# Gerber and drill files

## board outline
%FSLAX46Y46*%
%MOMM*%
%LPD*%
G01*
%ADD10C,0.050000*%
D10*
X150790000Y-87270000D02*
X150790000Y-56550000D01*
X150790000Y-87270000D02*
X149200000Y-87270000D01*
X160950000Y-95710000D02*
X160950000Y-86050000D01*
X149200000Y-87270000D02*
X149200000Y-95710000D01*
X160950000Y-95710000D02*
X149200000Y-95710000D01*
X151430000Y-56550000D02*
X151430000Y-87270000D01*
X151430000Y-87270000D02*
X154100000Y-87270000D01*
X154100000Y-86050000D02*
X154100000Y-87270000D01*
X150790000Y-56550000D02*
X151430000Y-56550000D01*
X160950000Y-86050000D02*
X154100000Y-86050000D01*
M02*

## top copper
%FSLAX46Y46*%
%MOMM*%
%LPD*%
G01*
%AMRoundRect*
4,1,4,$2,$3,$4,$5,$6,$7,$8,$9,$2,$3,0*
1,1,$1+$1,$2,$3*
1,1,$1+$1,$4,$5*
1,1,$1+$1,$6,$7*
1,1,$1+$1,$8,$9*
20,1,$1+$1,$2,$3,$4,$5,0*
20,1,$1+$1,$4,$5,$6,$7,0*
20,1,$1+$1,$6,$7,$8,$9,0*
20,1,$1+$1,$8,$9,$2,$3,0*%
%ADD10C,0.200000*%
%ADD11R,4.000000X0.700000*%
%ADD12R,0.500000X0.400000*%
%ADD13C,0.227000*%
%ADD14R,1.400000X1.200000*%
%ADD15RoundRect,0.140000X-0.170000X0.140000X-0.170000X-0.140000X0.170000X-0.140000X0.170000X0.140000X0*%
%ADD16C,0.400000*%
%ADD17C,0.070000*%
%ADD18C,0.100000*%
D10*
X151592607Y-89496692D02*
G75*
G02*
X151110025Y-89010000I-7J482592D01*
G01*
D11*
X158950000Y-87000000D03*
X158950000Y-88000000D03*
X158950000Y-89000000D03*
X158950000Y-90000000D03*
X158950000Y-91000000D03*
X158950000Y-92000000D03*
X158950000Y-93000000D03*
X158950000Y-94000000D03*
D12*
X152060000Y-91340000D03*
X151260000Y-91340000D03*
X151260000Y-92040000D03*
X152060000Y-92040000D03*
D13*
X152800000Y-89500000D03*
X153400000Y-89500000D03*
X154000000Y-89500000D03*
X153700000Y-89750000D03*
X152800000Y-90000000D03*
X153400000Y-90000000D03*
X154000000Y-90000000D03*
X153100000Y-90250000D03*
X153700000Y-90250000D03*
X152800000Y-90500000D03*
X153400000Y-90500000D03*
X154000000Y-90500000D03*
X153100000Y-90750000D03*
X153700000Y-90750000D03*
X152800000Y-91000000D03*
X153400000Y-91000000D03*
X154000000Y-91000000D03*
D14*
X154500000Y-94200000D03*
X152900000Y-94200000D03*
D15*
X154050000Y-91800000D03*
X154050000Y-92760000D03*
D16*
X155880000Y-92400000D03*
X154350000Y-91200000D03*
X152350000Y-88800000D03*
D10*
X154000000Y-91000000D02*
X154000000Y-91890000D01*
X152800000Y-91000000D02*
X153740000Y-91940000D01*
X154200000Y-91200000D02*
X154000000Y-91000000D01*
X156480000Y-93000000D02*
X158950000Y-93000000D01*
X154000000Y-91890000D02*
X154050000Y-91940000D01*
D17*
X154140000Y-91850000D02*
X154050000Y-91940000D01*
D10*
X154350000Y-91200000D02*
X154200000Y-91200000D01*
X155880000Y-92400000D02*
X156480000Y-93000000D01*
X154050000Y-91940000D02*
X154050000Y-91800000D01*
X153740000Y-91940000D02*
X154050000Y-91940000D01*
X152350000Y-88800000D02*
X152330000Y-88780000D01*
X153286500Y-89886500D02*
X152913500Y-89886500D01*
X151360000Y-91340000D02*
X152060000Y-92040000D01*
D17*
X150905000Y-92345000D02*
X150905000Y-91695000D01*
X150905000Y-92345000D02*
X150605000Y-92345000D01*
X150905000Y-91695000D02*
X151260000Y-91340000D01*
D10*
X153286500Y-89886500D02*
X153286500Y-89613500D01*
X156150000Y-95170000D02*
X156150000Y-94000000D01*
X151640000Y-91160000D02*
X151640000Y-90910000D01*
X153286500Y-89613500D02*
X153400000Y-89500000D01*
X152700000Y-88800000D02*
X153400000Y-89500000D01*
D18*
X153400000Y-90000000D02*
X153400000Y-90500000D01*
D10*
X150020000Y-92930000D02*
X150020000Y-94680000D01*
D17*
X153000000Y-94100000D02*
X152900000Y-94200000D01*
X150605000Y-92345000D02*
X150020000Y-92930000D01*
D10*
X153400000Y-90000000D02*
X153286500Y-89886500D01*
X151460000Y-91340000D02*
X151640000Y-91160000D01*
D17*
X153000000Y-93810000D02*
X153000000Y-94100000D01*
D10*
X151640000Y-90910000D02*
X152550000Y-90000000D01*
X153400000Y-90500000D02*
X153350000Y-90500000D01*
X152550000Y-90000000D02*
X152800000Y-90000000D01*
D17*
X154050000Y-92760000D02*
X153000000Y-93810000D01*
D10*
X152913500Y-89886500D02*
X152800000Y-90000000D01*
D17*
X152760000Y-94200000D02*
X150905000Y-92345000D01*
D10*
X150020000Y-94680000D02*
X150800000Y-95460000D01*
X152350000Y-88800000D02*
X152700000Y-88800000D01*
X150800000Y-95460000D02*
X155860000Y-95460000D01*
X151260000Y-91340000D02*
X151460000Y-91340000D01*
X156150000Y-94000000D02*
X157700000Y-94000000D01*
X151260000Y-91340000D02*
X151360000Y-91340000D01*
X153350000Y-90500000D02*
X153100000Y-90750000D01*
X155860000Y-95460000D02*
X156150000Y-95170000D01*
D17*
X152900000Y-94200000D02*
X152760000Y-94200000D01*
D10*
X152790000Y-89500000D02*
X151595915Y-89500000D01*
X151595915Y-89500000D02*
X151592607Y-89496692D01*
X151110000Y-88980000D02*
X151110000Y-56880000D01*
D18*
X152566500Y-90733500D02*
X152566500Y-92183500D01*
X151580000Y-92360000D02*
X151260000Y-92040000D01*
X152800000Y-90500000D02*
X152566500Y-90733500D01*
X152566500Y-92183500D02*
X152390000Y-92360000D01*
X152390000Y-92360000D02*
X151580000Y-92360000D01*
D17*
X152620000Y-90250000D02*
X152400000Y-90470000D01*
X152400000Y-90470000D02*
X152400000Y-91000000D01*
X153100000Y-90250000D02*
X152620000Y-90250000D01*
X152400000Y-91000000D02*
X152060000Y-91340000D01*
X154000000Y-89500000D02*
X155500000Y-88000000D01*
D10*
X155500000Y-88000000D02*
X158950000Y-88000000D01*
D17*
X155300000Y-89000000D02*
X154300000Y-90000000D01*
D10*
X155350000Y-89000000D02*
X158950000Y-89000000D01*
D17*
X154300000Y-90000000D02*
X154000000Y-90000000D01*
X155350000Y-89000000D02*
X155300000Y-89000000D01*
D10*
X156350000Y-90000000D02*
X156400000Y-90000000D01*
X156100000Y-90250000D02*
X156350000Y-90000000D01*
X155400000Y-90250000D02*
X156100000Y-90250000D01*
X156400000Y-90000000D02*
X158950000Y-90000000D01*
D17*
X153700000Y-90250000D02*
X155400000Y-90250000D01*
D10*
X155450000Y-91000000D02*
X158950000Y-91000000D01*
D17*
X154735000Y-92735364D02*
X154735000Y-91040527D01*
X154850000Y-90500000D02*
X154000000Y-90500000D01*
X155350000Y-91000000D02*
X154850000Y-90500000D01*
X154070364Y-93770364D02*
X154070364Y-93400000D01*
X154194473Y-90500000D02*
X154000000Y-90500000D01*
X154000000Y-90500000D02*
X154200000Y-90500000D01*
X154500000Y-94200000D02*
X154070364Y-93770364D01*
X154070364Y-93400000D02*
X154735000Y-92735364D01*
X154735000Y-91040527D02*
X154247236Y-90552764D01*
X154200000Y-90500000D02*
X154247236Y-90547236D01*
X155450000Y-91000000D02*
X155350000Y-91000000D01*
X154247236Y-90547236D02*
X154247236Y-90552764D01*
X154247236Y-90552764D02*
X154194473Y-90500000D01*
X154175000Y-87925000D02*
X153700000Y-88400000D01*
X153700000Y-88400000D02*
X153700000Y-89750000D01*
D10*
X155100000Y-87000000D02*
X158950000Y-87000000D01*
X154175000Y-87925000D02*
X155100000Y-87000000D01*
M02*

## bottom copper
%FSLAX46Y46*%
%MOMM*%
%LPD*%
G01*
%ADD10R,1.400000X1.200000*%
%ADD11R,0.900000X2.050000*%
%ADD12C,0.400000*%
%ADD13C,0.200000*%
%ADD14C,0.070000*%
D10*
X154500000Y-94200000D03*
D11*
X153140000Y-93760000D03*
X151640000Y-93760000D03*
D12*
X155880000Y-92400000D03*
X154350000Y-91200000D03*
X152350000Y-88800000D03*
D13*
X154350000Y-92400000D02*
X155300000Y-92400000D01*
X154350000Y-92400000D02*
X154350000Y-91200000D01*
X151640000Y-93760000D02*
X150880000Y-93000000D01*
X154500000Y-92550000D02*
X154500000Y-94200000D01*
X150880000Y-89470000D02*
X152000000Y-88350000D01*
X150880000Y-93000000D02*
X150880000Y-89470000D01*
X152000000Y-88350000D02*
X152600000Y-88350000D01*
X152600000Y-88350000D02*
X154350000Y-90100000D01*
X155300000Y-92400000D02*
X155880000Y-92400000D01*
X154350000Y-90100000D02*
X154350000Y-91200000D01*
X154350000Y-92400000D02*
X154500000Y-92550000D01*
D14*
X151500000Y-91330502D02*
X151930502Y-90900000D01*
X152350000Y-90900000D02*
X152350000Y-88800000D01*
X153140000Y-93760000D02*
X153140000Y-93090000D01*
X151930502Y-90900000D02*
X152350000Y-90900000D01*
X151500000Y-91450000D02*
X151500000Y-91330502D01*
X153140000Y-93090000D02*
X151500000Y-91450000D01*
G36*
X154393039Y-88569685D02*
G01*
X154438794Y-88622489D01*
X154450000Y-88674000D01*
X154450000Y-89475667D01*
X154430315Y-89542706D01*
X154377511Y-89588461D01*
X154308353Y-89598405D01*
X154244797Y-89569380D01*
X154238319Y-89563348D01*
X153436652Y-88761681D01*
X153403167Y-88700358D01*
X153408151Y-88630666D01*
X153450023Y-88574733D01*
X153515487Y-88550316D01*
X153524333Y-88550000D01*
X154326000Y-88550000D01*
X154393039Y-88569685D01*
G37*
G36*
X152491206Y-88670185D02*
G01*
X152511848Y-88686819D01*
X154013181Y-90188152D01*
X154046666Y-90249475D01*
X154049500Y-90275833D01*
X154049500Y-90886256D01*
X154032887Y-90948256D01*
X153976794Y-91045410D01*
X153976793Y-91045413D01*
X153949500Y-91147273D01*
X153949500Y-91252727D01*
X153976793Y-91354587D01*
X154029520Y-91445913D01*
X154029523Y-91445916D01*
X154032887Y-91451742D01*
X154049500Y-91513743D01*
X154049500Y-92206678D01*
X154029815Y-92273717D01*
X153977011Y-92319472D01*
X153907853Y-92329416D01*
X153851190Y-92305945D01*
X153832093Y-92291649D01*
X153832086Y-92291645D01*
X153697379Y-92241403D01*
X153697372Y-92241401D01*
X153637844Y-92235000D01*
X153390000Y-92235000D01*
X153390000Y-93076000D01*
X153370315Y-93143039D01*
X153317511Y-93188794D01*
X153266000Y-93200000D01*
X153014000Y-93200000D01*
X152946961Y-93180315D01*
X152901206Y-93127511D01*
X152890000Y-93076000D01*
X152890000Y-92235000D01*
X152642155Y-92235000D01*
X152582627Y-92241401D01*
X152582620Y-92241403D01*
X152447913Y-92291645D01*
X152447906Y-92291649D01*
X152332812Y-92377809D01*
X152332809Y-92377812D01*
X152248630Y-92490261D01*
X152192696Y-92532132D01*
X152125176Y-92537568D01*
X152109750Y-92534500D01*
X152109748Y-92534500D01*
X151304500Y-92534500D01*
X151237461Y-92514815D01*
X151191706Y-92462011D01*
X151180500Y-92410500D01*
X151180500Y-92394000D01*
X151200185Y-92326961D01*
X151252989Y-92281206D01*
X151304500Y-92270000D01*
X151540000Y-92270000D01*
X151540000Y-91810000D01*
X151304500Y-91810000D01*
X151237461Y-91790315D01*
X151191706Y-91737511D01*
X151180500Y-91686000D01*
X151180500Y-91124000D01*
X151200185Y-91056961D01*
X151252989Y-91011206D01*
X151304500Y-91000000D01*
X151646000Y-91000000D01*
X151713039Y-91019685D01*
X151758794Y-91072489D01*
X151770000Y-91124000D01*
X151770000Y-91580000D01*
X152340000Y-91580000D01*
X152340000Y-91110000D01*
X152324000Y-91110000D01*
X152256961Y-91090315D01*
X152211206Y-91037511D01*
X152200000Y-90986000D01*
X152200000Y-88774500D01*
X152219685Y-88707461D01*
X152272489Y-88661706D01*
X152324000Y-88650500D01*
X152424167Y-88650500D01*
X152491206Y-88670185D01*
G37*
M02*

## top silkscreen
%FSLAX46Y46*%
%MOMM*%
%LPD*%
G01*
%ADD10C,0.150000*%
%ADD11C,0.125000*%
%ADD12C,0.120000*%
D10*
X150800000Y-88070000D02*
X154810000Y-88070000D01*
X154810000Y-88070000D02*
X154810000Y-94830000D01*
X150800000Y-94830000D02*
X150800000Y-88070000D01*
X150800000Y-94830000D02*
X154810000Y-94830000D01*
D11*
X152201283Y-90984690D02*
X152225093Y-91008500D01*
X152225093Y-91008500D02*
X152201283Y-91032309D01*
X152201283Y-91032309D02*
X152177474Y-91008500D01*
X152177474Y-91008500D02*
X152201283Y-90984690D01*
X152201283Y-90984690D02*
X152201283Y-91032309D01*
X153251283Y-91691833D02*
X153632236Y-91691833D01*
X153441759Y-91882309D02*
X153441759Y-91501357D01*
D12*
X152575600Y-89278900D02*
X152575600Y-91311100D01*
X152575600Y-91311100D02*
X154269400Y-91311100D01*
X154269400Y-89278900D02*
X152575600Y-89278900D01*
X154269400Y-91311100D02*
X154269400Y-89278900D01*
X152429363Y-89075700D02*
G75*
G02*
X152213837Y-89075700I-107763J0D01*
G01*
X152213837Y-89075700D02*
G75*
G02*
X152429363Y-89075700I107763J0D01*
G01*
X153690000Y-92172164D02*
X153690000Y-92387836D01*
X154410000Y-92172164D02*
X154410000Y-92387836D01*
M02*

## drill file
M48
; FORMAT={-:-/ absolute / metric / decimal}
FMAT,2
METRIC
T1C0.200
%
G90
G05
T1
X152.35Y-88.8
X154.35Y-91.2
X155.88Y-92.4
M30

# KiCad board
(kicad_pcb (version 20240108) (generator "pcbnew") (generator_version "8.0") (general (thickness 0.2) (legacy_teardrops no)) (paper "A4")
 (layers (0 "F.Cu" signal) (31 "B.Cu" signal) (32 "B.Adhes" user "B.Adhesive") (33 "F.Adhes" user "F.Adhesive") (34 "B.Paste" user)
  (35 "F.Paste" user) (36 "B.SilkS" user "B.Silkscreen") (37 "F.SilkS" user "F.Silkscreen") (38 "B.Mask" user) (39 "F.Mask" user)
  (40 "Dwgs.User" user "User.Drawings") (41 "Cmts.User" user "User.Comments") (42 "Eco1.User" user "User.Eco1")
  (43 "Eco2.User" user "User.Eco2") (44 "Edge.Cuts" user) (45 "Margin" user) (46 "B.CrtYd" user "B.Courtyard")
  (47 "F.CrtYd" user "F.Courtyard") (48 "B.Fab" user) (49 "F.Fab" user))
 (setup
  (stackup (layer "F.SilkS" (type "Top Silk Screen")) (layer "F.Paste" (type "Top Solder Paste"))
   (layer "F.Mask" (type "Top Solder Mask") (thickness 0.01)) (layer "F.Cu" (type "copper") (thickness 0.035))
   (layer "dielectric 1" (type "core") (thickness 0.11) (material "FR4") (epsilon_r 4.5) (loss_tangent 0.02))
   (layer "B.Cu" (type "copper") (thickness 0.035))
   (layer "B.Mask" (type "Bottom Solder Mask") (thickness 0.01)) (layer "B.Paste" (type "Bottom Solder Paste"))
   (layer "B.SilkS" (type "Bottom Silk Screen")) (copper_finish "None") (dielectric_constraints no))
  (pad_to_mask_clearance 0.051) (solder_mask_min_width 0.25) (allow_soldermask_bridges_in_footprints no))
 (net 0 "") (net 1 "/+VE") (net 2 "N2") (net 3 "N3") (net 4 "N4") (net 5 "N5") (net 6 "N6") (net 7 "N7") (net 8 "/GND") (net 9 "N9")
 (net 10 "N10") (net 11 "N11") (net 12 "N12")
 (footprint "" (layer "F.Cu") (at 154.5 94.2)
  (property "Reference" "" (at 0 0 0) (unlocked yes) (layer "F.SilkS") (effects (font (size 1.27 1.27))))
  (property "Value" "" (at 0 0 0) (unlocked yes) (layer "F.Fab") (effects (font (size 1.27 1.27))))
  (pad "2" smd rect (at 0 0 270) (size 1.2 1.4) (layers "B.Cu" "B.Paste" "B.Mask") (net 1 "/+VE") (solder_mask_margin 0.102)))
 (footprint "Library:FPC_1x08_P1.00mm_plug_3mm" (layer "F.Cu") (at 156.95 90.5)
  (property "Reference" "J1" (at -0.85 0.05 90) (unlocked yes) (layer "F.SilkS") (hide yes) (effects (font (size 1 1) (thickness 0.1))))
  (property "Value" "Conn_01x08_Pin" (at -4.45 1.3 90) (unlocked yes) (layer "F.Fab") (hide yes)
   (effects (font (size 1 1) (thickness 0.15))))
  (pad "1" connect rect (at 2 -3.5) (size 4 0.7) (layers "F.Cu" "F.Mask") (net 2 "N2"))
  (pad "2" connect rect (at 2 -2.5) (size 4 0.7) (layers "F.Cu" "F.Mask") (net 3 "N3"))
  (pad "3" connect rect (at 2 -1.5) (size 4 0.7) (layers "F.Cu" "F.Mask") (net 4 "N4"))
  (pad "4" connect rect (at 2 -0.5) (size 4 0.7) (layers "F.Cu" "F.Mask") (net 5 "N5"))
  (pad "5" connect rect (at 2 0.5) (size 4 0.7) (layers "F.Cu" "F.Mask") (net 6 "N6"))
  (pad "6" connect rect (at 2 1.5) (size 4 0.7) (layers "F.Cu" "F.Mask") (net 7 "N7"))
  (pad "7" connect rect (at 2 2.5) (size 4 0.7) (layers "F.Cu" "F.Mask") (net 1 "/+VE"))
  (pad "8" connect rect (at 2 3.5) (size 4 0.7) (layers "F.Cu" "F.Mask") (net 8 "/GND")))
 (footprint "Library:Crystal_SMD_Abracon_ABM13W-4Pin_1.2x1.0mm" (layer "F.Cu") (at 151.66 91.69 180)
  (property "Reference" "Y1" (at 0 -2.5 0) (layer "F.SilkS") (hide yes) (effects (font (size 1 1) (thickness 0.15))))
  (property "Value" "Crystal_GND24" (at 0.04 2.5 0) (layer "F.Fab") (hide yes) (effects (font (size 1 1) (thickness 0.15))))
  (pad "1" smd rect (at -0.4 0.35 180) (size 0.5 0.4) (layers "F.Cu" "F.Paste" "F.Mask") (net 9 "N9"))
  (pad "2" smd rect (at 0.4 0.35 180) (size 0.5 0.4) (layers "F.Cu" "F.Paste" "F.Mask") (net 8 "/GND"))
  (pad "3" smd rect (at 0.4 -0.35 180) (size 0.5 0.4) (layers "F.Cu" "F.Paste" "F.Mask") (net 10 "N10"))
  (pad "4" smd rect (at -0.4 -0.35 180) (size 0.5 0.4) (layers "F.Cu" "F.Paste" "F.Mask") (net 8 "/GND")))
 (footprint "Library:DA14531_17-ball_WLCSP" (layer "F.Cu") (at 153.422 90.295)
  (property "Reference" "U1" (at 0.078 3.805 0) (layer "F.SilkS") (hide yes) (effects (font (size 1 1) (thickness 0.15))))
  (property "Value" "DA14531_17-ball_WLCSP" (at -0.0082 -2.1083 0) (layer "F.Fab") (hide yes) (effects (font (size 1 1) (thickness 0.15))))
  (fp_line (start -0.8464 -1.0161) (end -0.8464 1.0161) (stroke (width 0.12) (type solid)) (layer "F.SilkS"))
  (fp_line (start -0.8464 1.0161) (end 0.8474 1.0161) (stroke (width 0.12) (type solid)) (layer "F.SilkS"))
  (fp_line (start 0.8474 -1.0161) (end -0.8464 -1.0161) (stroke (width 0.12) (type solid)) (layer "F.SilkS"))
  (fp_line (start 0.8474 1.0161) (end 0.8474 -1.0161) (stroke (width 0.12) (type solid)) (layer "F.SilkS"))
  (fp_circle (center -1.1004 -1.2193) (end -1.0242 -1.1431) (stroke (width 0.12) (type solid)) (fill none) (layer "F.SilkS"))
  (pad "A1" smd circle (at -0.622 -0.795) (size 0.227 0.227) (layers "F.Cu" "F.Paste" "F.Mask") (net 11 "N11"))
  (pad "A3" smd circle (at -0.022 -0.795) (size 0.227 0.227) (layers "F.Cu" "F.Paste" "F.Mask") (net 8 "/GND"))
  (pad "A5" smd circle (at 0.578 -0.795) (size 0.227 0.227) (layers "F.Cu" "F.Paste" "F.Mask") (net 3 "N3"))
  (pad "B4" smd circle (at 0.278 -0.545) (size 0.227 0.227) (layers "F.Cu" "F.Paste" "F.Mask") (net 2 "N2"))
  (pad "C1" smd circle (at -0.622 -0.295) (size 0.227 0.227) (layers "F.Cu" "F.Paste" "F.Mask") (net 8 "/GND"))
  (pad "C3" smd circle (at -0.022 -0.295) (size 0.227 0.227) (layers "F.Cu" "F.Paste" "F.Mask") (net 8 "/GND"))
  (pad "C5" smd circle (at 0.578 -0.295) (size 0.227 0.227) (layers "F.Cu" "F.Paste" "F.Mask") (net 4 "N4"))
  (pad "D2" smd circle (at -0.322 -0.045) (size 0.227 0.227) (layers "F.Cu" "F.Paste" "F.Mask") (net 9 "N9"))
  (pad "D4" smd circle (at 0.278 -0.045) (size 0.227 0.227) (layers "F.Cu" "F.Paste" "F.Mask") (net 5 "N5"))
  (pad "E1" smd circle (at -0.622 0.205) (size 0.227 0.227) (layers "F.Cu" "F.Paste" "F.Mask") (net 10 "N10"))
  (pad "E3" smd circle (at -0.022 0.205) (size 0.227 0.227) (layers "F.Cu" "F.Paste" "F.Mask") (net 8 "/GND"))
  (pad "E5" smd circle (at 0.578 0.205) (size 0.227 0.227) (layers "F.Cu" "F.Paste" "F.Mask") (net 6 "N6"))
  (pad "F2" smd circle (at -0.322 0.455) (size 0.227 0.227) (layers "F.Cu" "F.Paste" "F.Mask") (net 8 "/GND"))
  (pad "F4" smd circle (at 0.278 0.455) (size 0.227 0.227) (layers "F.Cu" "F.Paste" "F.Mask") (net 7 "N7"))
  (pad "G1" smd circle (at -0.622 0.705) (size 0.227 0.227) (layers "F.Cu" "F.Paste" "F.Mask") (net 1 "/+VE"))
  (pad "G3" smd circle (at -0.022 0.705) (size 0.227 0.227) (layers "F.Cu" "F.Paste" "F.Mask") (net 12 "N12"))
  (pad "G5" smd circle (at 0.578 0.705) (size 0.227 0.227) (layers "F.Cu" "F.Paste" "F.Mask") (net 1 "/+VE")))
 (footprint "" (layer "F.Cu") (at 154.5 94.2)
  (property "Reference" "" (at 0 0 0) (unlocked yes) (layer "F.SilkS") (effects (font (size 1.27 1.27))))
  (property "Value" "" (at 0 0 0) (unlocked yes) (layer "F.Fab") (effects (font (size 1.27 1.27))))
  (pad "2" smd rect (at 0 0 270) (size 1.2 1.4) (layers "F.Cu" "F.Paste" "F.Mask") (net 6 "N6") (solder_mask_margin 0.102)))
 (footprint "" (layer "F.Cu") (at 152.9 94.2)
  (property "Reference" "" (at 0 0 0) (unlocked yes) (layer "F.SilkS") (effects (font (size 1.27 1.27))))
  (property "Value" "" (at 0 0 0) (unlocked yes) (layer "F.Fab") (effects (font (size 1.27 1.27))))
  (pad "2" smd rect (at 0 0 270) (size 1.2 1.4) (layers "F.Cu" "F.Paste" "F.Mask") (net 8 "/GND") (solder_mask_margin 0.102)))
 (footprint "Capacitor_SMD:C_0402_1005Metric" (layer "F.Cu") (at 154.05 92.28 -90)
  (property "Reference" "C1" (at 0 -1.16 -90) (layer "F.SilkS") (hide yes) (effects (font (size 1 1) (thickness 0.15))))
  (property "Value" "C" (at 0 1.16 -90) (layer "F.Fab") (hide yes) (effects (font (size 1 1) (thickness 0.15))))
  (fp_line (start -0.107836 0.36) (end 0.107836 0.36) (stroke (width 0.12) (type solid)) (layer "F.SilkS"))
  (fp_line (start -0.107836 -0.36) (end 0.107836 -0.36) (stroke (width 0.12) (type solid)) (layer "F.SilkS"))
  (pad "1" smd roundrect (at -0.48 0 270) (size 0.56 0.62) (layers "F.Cu" "F.Paste" "F.Mask") (roundrect_rratio 0.25) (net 1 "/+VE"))
  (pad "2" smd roundrect (at 0.48 0 270) (size 0.56 0.62) (layers "F.Cu" "F.Paste" "F.Mask") (roundrect_rratio 0.25) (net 8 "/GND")))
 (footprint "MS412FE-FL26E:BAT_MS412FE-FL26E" (layer "B.Cu") (at 152.39 90.035 -90)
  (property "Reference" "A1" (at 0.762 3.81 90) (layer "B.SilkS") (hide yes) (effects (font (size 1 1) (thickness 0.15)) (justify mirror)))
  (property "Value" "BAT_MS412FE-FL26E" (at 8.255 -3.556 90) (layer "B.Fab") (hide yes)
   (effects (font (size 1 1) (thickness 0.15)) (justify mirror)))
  (pad "N1" smd rect (at 3.725 -0.75 270) (size 2.05 0.9) (layers "B.Cu" "B.Paste" "B.Mask") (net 8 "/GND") (solder_mask_margin 0.102))
  (pad "P1" smd rect (at 3.725 0.75 270) (size 2.05 0.9) (layers "B.Cu" "B.Paste" "B.Mask") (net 1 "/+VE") (solder_mask_margin 0.102)))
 (gr_arc (start 151.592607 89.496692) (mid 151.249908 89.353892) (end 151.11 89.01) (stroke (width 0.2) (type default)) (layer "F.Cu")
  (net 11))
 (gr_line (start 150.8 88.07) (end 154.81 88.07) (stroke (width 0.15) (type default)) (layer "F.SilkS"))
 (gr_line (start 154.81 88.07) (end 154.81 94.83) (stroke (width 0.15) (type default)) (layer "F.SilkS"))
 (gr_line (start 150.8 94.83) (end 150.8 88.07) (stroke (width 0.15) (type default)) (layer "F.SilkS"))
 (gr_line (start 150.8 94.83) (end 154.81 94.83) (stroke (width 0.15) (type default)) (layer "F.SilkS"))
 (gr_line (start 150.79 87.27) (end 150.79 56.55) (stroke (width 0.05) (type default)) (layer "Edge.Cuts"))
 (gr_line (start 150.79 87.27) (end 149.2 87.27) (stroke (width 0.05) (type default)) (layer "Edge.Cuts"))
 (gr_line (start 160.95 95.71) (end 160.95 86.05) (stroke (width 0.05) (type default)) (layer "Edge.Cuts"))
 (gr_line (start 149.2 87.27) (end 149.2 95.71) (stroke (width 0.05) (type default)) (layer "Edge.Cuts"))
 (gr_line (start 160.95 95.71) (end 149.2 95.71) (stroke (width 0.05) (type default)) (layer "Edge.Cuts"))
 (gr_line (start 151.43 56.55) (end 151.43 87.27) (stroke (width 0.05) (type default)) (layer "Edge.Cuts"))
 (gr_line (start 151.43 87.27) (end 154.1 87.27) (stroke (width 0.05) (type default)) (layer "Edge.Cuts"))
 (gr_line (start 154.1 86.05) (end 154.1 87.27) (stroke (width 0.05) (type default)) (layer "Edge.Cuts"))
 (gr_line (start 150.79 56.55) (end 151.43 56.55) (stroke (width 0.05) (type default)) (layer "Edge.Cuts"))
 (gr_line (start 160.95 86.05) (end 154.1 86.05) (stroke (width 0.05) (type default)) (layer "Edge.Cuts"))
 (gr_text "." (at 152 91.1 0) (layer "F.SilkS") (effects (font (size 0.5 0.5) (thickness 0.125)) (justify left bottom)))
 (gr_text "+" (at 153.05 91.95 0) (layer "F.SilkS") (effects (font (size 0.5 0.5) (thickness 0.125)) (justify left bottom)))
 (segment (start 154 91) (end 154 91.89) (width 0.2) (layer "F.Cu") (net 1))
 (segment (start 152.8 91) (end 153.74 91.94) (width 0.2) (layer "F.Cu") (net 1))
 (segment (start 154.2 91.2) (end 154 91) (width 0.2) (layer "F.Cu") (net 1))
 (segment (start 156.48 93) (end 158.95 93) (width 0.2) (layer "F.Cu") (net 1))
 (segment (start 154 91.89) (end 154.05 91.94) (width 0.2) (layer "F.Cu") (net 1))
 (segment (start 154.14 91.85) (end 154.05 91.94) (width 0.07) (layer "F.Cu") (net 1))
 (segment (start 154.35 91.2) (end 154.2 91.2) (width 0.2) (layer "F.Cu") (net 1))
 (segment (start 155.88 92.4) (end 156.48 93) (width 0.2) (layer "F.Cu") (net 1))
 (segment (start 154.05 91.94) (end 154.05 91.8) (width 0.2) (layer "F.Cu") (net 1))
 (segment (start 153.74 91.94) (end 154.05 91.94) (width 0.2) (layer "F.Cu") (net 1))
 (via (at 155.88 92.4) (size 0.4) (drill 0.2) (layers "F.Cu" "B.Cu") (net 1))
 (via (at 154.35 91.2) (size 0.4) (drill 0.2) (layers "F.Cu" "B.Cu") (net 1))
 (segment (start 154.35 92.4) (end 155.3 92.4) (width 0.2) (layer "B.Cu") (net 1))
 (segment (start 154.35 92.4) (end 154.35 91.2) (width 0.2) (layer "B.Cu") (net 1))
 (segment (start 151.64 93.76) (end 150.88 93) (width 0.2) (layer "B.Cu") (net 1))
 (segment (start 154.5 92.55) (end 154.5 94.2) (width 0.2) (layer "B.Cu") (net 1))
 (segment (start 150.88 89.47) (end 152 88.35) (width 0.2) (layer "B.Cu") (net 1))
 (segment (start 150.88 93) (end 150.88 89.47) (width 0.2) (layer "B.Cu") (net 1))
 (segment (start 152 88.35) (end 152.6 88.35) (width 0.2) (layer "B.Cu") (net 1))
 (segment (start 152.6 88.35) (end 154.35 90.1) (width 0.2) (layer "B.Cu") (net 1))
 (segment (start 155.3 92.4) (end 155.88 92.4) (width 0.2) (layer "B.Cu") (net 1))
 (segment (start 154.35 90.1) (end 154.35 91.2) (width 0.2) (layer "B.Cu") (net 1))
 (segment (start 154.35 92.4) (end 154.5 92.55) (width 0.2) (layer "B.Cu") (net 1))
 (segment (start 152.35 88.8) (end 152.33 88.78) (width 0.2) (layer "F.Cu") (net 8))
 (segment (start 153.2865 89.8865) (end 152.9135 89.8865) (width 0.2) (layer "F.Cu") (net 8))
 (segment (start 151.36 91.34) (end 152.06 92.04) (width 0.2) (layer "F.Cu") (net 8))
 (segment (start 150.905 92.345) (end 150.905 91.695) (width 0.07) (layer "F.Cu") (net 8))
 (segment (start 150.905 92.345) (end 150.605 92.345) (width 0.07) (layer "F.Cu") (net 8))
 (segment (start 150.905 91.695) (end 151.26 91.34) (width 0.07) (layer "F.Cu") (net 8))
 (segment (start 153.2865 89.8865) (end 153.2865 89.6135) (width 0.2) (layer "F.Cu") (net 8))
 (segment (start 156.15 95.17) (end 156.15 94) (width 0.2) (layer "F.Cu") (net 8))
 (segment (start 151.64 91.16) (end 151.64 90.91) (width 0.2) (layer "F.Cu") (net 8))
 (segment (start 153.2865 89.6135) (end 153.4 89.5) (width 0.2) (layer "F.Cu") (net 8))
 (segment (start 152.7 88.8) (end 153.4 89.5) (width 0.2) (layer "F.Cu") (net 8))
 (segment (start 153.4 90) (end 153.4 90.5) (width 0.1) (layer "F.Cu") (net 8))
 (segment (start 150.02 92.93) (end 150.02 94.68) (width 0.2) (layer "F.Cu") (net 8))
 (segment (start 153 94.1) (end 152.9 94.2) (width 0.07) (layer "F.Cu") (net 8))
 (segment (start 150.605 92.345) (end 150.02 92.93) (width 0.07) (layer "F.Cu") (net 8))
 (segment (start 153.4 90) (end 153.2865 89.8865) (width 0.2) (layer "F.Cu") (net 8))
 (segment (start 151.46 91.34) (end 151.64 91.16) (width 0.2) (layer "F.Cu") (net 8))
 (segment (start 153 93.81) (end 153 94.1) (width 0.07) (layer "F.Cu") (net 8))
 (segment (start 151.64 90.91) (end 152.55 90) (width 0.2) (layer "F.Cu") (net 8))
 (segment (start 153.4 90.5) (end 153.35 90.5) (width 0.2) (layer "F.Cu") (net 8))
 (segment (start 152.55 90) (end 152.8 90) (width 0.2) (layer "F.Cu") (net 8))
 (segment (start 154.05 92.76) (end 153 93.81) (width 0.07) (layer "F.Cu") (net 8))
 (segment (start 152.9135 89.8865) (end 152.8 90) (width 0.2) (layer "F.Cu") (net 8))
 (segment (start 152.76 94.2) (end 150.905 92.345) (width 0.07) (layer "F.Cu") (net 8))
 (segment (start 150.02 94.68) (end 150.8 95.46) (width 0.2) (layer "F.Cu") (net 8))
 (segment (start 152.35 88.8) (end 152.7 88.8) (width 0.2) (layer "F.Cu") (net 8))
 (segment (start 150.8 95.46) (end 155.86 95.46) (width 0.2) (layer "F.Cu") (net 8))
 (segment (start 151.26 91.34) (end 151.46 91.34) (width 0.2) (layer "F.Cu") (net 8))
 (segment (start 156.15 94) (end 157.7 94) (width 0.2) (layer "F.Cu") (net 8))
 (segment (start 151.26 91.34) (end 151.36 91.34) (width 0.2) (layer "F.Cu") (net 8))
 (segment (start 153.35 90.5) (end 153.1 90.75) (width 0.2) (layer "F.Cu") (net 8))
 (segment (start 155.86 95.46) (end 156.15 95.17) (width 0.2) (layer "F.Cu") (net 8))
 (segment (start 152.9 94.2) (end 152.76 94.2) (width 0.07) (layer "F.Cu") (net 8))
 (via (at 152.35 88.8) (size 0.4) (drill 0.2) (layers "F.Cu" "B.Cu") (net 8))
 (segment (start 151.5 91.330502) (end 151.930502 90.9) (width 0.07) (layer "B.Cu") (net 8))
 (segment (start 152.35 90.9) (end 152.35 88.8) (width 0.07) (layer "B.Cu") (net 8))
 (segment (start 153.14 93.76) (end 153.14 93.09) (width 0.07) (layer "B.Cu") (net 8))
 (segment (start 151.930502 90.9) (end 152.35 90.9) (width 0.07) (layer "B.Cu") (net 8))
 (segment (start 151.5 91.45) (end 151.5 91.330502) (width 0.07) (layer "B.Cu") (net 8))
 (segment (start 153.14 93.09) (end 151.5 91.45) (width 0.07) (layer "B.Cu") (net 8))
 (segment (start 152.79 89.5) (end 151.595915 89.5) (width 0.2) (layer "F.Cu") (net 11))
 (segment (start 151.595915 89.5) (end 151.592607 89.496692) (width 0.2) (layer "F.Cu") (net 11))
 (segment (start 151.11 88.98) (end 151.11 56.88) (width 0.2) (layer "F.Cu") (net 11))
 (segment (start 152.5665 90.7335) (end 152.5665 92.1835) (width 0.1) (layer "F.Cu") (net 10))
 (segment (start 151.58 92.36) (end 151.26 92.04) (width 0.1) (layer "F.Cu") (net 10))
 (segment (start 152.8 90.5) (end 152.5665 90.7335) (width 0.1) (layer "F.Cu") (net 10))
 (segment (start 152.5665 92.1835) (end 152.39 92.36) (width 0.1) (layer "F.Cu") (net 10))
 (segment (start 152.39 92.36) (end 151.58 92.36) (width 0.1) (layer "F.Cu") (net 10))
 (segment (start 152.62 90.25) (end 152.4 90.47) (width 0.07) (layer "F.Cu") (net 9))
 (segment (start 152.4 90.47) (end 152.4 91) (width 0.07) (layer "F.Cu") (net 9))
 (segment (start 153.1 90.25) (end 152.62 90.25) (width 0.07) (layer "F.Cu") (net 9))
 (segment (start 152.4 91) (end 152.06 91.34) (width 0.07) (layer "F.Cu") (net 9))
 (segment (start 154 89.5) (end 155.5 88) (width 0.07) (layer "F.Cu") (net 3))
 (segment (start 155.5 88) (end 158.95 88) (width 0.2) (layer "F.Cu") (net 3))
 (segment (start 155.3 89) (end 154.3 90) (width 0.07) (layer "F.Cu") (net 4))
 (segment (start 155.35 89) (end 158.95 89) (width 0.2) (layer "F.Cu") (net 4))
 (segment (start 154.3 90) (end 154 90) (width 0.07) (layer "F.Cu") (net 4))
 (segment (start 155.35 89) (end 155.3 89) (width 0.07) (layer "F.Cu") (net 4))
 (segment (start 156.35 90) (end 156.4 90) (width 0.2) (layer "F.Cu") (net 5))
 (segment (start 156.1 90.25) (end 156.35 90) (width 0.2) (layer "F.Cu") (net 5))
 (segment (start 155.4 90.25) (end 156.1 90.25) (width 0.2) (layer "F.Cu") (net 5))
 (segment (start 156.4 90) (end 158.95 90) (width 0.2) (layer "F.Cu") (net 5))
 (segment (start 153.7 90.25) (end 155.4 90.25) (width 0.07) (layer "F.Cu") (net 5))
 (segment (start 155.45 91) (end 158.95 91) (width 0.2) (layer "F.Cu") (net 6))
 (segment (start 154.735 92.735364) (end 154.735 91.040527) (width 0.07) (layer "F.Cu") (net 6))
 (segment (start 154.85 90.5) (end 154 90.5) (width 0.07) (layer "F.Cu") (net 6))
 (segment (start 155.35 91) (end 154.85 90.5) (width 0.07) (layer "F.Cu") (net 6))
 (segment (start 154.070364 93.770364) (end 154.070364 93.4) (width 0.07) (layer "F.Cu") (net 6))
 (segment (start 154.194473 90.5) (end 154 90.5) (width 0.07) (layer "F.Cu") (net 6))
 (segment (start 154 90.5) (end 154.2 90.5) (width 0.07) (layer "F.Cu") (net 6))
 (segment (start 154.5 94.2) (end 154.070364 93.770364) (width 0.07) (layer "F.Cu") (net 6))
 (segment (start 154.070364 93.4) (end 154.735 92.735364) (width 0.07) (layer "F.Cu") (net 6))
 (segment (start 154.735 91.040527) (end 154.247236 90.552764) (width 0.07) (layer "F.Cu") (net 6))
 (segment (start 154.2 90.5) (end 154.247236 90.547236) (width 0.07) (layer "F.Cu") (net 6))
 (segment (start 155.45 91) (end 155.35 91) (width 0.07) (layer "F.Cu") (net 6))
 (segment (start 154.247236 90.547236) (end 154.247236 90.552764) (width 0.07) (layer "F.Cu") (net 6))
 (segment (start 154.247236 90.552764) (end 154.194473 90.5) (width 0.07) (layer "F.Cu") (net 6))
 (segment (start 154.175 87.925) (end 153.7 88.4) (width 0.07) (layer "F.Cu") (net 2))
 (segment (start 153.7 88.4) (end 153.7 89.75) (width 0.07) (layer "F.Cu") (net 2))
 (segment (start 155.1 87) (end 158.95 87) (width 0.2) (layer "F.Cu") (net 2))
 (segment (start 154.175 87.925) (end 155.1 87) (width 0.2) (layer "F.Cu") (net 2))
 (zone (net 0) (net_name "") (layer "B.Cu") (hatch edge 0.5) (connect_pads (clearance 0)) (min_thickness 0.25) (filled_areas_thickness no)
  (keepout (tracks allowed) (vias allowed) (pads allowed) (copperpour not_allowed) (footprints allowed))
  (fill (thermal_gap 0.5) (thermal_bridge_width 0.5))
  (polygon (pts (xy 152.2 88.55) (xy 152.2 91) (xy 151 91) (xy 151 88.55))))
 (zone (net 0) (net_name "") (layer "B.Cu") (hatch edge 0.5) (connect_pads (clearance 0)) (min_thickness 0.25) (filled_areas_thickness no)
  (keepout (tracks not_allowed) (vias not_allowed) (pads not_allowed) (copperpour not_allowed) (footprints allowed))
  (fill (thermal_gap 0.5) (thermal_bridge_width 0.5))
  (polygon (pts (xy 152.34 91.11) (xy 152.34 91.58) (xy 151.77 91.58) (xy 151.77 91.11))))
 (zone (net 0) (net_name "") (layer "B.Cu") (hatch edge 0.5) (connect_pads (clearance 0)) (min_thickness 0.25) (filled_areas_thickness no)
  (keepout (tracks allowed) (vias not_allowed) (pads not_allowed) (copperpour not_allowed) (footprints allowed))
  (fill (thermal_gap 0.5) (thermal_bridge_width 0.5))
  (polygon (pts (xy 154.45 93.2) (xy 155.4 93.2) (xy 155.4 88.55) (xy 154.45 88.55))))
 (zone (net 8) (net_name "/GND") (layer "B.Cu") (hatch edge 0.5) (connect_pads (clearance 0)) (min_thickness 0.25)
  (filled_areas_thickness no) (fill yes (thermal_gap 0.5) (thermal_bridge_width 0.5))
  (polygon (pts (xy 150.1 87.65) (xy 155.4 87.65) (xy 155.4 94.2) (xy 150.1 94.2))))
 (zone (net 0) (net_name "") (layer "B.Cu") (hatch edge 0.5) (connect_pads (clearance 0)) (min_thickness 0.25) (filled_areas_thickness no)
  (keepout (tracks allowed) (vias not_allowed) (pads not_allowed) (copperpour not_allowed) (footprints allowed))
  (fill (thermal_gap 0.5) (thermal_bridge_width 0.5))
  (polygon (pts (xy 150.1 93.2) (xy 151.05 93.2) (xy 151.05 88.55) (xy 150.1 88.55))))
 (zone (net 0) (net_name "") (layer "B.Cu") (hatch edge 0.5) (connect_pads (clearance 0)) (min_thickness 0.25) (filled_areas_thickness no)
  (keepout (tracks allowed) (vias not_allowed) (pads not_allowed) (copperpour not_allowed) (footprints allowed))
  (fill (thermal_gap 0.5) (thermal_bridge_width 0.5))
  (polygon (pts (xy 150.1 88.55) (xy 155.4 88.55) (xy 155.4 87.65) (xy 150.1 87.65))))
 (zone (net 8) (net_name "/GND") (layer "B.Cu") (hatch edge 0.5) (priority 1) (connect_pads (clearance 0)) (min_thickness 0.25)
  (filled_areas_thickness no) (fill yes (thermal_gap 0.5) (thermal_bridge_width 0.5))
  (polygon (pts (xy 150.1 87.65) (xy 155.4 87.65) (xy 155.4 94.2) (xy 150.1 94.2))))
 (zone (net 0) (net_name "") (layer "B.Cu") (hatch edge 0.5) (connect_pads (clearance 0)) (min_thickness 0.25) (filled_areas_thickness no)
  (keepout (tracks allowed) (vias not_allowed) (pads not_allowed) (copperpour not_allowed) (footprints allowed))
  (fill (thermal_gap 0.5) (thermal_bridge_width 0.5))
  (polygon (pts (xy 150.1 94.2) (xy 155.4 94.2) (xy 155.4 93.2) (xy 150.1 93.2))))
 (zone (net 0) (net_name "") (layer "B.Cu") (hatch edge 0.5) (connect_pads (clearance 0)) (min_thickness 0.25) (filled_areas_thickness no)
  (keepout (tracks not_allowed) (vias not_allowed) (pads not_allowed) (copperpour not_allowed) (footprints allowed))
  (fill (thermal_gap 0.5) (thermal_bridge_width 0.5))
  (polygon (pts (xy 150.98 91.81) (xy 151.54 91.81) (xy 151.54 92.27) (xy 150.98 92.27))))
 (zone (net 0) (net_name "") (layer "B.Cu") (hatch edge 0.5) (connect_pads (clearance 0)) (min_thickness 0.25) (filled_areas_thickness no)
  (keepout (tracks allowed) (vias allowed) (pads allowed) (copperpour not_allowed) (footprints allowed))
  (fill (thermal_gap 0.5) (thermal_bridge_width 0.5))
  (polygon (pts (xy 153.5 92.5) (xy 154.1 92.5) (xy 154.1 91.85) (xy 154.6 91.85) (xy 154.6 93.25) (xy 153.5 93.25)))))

